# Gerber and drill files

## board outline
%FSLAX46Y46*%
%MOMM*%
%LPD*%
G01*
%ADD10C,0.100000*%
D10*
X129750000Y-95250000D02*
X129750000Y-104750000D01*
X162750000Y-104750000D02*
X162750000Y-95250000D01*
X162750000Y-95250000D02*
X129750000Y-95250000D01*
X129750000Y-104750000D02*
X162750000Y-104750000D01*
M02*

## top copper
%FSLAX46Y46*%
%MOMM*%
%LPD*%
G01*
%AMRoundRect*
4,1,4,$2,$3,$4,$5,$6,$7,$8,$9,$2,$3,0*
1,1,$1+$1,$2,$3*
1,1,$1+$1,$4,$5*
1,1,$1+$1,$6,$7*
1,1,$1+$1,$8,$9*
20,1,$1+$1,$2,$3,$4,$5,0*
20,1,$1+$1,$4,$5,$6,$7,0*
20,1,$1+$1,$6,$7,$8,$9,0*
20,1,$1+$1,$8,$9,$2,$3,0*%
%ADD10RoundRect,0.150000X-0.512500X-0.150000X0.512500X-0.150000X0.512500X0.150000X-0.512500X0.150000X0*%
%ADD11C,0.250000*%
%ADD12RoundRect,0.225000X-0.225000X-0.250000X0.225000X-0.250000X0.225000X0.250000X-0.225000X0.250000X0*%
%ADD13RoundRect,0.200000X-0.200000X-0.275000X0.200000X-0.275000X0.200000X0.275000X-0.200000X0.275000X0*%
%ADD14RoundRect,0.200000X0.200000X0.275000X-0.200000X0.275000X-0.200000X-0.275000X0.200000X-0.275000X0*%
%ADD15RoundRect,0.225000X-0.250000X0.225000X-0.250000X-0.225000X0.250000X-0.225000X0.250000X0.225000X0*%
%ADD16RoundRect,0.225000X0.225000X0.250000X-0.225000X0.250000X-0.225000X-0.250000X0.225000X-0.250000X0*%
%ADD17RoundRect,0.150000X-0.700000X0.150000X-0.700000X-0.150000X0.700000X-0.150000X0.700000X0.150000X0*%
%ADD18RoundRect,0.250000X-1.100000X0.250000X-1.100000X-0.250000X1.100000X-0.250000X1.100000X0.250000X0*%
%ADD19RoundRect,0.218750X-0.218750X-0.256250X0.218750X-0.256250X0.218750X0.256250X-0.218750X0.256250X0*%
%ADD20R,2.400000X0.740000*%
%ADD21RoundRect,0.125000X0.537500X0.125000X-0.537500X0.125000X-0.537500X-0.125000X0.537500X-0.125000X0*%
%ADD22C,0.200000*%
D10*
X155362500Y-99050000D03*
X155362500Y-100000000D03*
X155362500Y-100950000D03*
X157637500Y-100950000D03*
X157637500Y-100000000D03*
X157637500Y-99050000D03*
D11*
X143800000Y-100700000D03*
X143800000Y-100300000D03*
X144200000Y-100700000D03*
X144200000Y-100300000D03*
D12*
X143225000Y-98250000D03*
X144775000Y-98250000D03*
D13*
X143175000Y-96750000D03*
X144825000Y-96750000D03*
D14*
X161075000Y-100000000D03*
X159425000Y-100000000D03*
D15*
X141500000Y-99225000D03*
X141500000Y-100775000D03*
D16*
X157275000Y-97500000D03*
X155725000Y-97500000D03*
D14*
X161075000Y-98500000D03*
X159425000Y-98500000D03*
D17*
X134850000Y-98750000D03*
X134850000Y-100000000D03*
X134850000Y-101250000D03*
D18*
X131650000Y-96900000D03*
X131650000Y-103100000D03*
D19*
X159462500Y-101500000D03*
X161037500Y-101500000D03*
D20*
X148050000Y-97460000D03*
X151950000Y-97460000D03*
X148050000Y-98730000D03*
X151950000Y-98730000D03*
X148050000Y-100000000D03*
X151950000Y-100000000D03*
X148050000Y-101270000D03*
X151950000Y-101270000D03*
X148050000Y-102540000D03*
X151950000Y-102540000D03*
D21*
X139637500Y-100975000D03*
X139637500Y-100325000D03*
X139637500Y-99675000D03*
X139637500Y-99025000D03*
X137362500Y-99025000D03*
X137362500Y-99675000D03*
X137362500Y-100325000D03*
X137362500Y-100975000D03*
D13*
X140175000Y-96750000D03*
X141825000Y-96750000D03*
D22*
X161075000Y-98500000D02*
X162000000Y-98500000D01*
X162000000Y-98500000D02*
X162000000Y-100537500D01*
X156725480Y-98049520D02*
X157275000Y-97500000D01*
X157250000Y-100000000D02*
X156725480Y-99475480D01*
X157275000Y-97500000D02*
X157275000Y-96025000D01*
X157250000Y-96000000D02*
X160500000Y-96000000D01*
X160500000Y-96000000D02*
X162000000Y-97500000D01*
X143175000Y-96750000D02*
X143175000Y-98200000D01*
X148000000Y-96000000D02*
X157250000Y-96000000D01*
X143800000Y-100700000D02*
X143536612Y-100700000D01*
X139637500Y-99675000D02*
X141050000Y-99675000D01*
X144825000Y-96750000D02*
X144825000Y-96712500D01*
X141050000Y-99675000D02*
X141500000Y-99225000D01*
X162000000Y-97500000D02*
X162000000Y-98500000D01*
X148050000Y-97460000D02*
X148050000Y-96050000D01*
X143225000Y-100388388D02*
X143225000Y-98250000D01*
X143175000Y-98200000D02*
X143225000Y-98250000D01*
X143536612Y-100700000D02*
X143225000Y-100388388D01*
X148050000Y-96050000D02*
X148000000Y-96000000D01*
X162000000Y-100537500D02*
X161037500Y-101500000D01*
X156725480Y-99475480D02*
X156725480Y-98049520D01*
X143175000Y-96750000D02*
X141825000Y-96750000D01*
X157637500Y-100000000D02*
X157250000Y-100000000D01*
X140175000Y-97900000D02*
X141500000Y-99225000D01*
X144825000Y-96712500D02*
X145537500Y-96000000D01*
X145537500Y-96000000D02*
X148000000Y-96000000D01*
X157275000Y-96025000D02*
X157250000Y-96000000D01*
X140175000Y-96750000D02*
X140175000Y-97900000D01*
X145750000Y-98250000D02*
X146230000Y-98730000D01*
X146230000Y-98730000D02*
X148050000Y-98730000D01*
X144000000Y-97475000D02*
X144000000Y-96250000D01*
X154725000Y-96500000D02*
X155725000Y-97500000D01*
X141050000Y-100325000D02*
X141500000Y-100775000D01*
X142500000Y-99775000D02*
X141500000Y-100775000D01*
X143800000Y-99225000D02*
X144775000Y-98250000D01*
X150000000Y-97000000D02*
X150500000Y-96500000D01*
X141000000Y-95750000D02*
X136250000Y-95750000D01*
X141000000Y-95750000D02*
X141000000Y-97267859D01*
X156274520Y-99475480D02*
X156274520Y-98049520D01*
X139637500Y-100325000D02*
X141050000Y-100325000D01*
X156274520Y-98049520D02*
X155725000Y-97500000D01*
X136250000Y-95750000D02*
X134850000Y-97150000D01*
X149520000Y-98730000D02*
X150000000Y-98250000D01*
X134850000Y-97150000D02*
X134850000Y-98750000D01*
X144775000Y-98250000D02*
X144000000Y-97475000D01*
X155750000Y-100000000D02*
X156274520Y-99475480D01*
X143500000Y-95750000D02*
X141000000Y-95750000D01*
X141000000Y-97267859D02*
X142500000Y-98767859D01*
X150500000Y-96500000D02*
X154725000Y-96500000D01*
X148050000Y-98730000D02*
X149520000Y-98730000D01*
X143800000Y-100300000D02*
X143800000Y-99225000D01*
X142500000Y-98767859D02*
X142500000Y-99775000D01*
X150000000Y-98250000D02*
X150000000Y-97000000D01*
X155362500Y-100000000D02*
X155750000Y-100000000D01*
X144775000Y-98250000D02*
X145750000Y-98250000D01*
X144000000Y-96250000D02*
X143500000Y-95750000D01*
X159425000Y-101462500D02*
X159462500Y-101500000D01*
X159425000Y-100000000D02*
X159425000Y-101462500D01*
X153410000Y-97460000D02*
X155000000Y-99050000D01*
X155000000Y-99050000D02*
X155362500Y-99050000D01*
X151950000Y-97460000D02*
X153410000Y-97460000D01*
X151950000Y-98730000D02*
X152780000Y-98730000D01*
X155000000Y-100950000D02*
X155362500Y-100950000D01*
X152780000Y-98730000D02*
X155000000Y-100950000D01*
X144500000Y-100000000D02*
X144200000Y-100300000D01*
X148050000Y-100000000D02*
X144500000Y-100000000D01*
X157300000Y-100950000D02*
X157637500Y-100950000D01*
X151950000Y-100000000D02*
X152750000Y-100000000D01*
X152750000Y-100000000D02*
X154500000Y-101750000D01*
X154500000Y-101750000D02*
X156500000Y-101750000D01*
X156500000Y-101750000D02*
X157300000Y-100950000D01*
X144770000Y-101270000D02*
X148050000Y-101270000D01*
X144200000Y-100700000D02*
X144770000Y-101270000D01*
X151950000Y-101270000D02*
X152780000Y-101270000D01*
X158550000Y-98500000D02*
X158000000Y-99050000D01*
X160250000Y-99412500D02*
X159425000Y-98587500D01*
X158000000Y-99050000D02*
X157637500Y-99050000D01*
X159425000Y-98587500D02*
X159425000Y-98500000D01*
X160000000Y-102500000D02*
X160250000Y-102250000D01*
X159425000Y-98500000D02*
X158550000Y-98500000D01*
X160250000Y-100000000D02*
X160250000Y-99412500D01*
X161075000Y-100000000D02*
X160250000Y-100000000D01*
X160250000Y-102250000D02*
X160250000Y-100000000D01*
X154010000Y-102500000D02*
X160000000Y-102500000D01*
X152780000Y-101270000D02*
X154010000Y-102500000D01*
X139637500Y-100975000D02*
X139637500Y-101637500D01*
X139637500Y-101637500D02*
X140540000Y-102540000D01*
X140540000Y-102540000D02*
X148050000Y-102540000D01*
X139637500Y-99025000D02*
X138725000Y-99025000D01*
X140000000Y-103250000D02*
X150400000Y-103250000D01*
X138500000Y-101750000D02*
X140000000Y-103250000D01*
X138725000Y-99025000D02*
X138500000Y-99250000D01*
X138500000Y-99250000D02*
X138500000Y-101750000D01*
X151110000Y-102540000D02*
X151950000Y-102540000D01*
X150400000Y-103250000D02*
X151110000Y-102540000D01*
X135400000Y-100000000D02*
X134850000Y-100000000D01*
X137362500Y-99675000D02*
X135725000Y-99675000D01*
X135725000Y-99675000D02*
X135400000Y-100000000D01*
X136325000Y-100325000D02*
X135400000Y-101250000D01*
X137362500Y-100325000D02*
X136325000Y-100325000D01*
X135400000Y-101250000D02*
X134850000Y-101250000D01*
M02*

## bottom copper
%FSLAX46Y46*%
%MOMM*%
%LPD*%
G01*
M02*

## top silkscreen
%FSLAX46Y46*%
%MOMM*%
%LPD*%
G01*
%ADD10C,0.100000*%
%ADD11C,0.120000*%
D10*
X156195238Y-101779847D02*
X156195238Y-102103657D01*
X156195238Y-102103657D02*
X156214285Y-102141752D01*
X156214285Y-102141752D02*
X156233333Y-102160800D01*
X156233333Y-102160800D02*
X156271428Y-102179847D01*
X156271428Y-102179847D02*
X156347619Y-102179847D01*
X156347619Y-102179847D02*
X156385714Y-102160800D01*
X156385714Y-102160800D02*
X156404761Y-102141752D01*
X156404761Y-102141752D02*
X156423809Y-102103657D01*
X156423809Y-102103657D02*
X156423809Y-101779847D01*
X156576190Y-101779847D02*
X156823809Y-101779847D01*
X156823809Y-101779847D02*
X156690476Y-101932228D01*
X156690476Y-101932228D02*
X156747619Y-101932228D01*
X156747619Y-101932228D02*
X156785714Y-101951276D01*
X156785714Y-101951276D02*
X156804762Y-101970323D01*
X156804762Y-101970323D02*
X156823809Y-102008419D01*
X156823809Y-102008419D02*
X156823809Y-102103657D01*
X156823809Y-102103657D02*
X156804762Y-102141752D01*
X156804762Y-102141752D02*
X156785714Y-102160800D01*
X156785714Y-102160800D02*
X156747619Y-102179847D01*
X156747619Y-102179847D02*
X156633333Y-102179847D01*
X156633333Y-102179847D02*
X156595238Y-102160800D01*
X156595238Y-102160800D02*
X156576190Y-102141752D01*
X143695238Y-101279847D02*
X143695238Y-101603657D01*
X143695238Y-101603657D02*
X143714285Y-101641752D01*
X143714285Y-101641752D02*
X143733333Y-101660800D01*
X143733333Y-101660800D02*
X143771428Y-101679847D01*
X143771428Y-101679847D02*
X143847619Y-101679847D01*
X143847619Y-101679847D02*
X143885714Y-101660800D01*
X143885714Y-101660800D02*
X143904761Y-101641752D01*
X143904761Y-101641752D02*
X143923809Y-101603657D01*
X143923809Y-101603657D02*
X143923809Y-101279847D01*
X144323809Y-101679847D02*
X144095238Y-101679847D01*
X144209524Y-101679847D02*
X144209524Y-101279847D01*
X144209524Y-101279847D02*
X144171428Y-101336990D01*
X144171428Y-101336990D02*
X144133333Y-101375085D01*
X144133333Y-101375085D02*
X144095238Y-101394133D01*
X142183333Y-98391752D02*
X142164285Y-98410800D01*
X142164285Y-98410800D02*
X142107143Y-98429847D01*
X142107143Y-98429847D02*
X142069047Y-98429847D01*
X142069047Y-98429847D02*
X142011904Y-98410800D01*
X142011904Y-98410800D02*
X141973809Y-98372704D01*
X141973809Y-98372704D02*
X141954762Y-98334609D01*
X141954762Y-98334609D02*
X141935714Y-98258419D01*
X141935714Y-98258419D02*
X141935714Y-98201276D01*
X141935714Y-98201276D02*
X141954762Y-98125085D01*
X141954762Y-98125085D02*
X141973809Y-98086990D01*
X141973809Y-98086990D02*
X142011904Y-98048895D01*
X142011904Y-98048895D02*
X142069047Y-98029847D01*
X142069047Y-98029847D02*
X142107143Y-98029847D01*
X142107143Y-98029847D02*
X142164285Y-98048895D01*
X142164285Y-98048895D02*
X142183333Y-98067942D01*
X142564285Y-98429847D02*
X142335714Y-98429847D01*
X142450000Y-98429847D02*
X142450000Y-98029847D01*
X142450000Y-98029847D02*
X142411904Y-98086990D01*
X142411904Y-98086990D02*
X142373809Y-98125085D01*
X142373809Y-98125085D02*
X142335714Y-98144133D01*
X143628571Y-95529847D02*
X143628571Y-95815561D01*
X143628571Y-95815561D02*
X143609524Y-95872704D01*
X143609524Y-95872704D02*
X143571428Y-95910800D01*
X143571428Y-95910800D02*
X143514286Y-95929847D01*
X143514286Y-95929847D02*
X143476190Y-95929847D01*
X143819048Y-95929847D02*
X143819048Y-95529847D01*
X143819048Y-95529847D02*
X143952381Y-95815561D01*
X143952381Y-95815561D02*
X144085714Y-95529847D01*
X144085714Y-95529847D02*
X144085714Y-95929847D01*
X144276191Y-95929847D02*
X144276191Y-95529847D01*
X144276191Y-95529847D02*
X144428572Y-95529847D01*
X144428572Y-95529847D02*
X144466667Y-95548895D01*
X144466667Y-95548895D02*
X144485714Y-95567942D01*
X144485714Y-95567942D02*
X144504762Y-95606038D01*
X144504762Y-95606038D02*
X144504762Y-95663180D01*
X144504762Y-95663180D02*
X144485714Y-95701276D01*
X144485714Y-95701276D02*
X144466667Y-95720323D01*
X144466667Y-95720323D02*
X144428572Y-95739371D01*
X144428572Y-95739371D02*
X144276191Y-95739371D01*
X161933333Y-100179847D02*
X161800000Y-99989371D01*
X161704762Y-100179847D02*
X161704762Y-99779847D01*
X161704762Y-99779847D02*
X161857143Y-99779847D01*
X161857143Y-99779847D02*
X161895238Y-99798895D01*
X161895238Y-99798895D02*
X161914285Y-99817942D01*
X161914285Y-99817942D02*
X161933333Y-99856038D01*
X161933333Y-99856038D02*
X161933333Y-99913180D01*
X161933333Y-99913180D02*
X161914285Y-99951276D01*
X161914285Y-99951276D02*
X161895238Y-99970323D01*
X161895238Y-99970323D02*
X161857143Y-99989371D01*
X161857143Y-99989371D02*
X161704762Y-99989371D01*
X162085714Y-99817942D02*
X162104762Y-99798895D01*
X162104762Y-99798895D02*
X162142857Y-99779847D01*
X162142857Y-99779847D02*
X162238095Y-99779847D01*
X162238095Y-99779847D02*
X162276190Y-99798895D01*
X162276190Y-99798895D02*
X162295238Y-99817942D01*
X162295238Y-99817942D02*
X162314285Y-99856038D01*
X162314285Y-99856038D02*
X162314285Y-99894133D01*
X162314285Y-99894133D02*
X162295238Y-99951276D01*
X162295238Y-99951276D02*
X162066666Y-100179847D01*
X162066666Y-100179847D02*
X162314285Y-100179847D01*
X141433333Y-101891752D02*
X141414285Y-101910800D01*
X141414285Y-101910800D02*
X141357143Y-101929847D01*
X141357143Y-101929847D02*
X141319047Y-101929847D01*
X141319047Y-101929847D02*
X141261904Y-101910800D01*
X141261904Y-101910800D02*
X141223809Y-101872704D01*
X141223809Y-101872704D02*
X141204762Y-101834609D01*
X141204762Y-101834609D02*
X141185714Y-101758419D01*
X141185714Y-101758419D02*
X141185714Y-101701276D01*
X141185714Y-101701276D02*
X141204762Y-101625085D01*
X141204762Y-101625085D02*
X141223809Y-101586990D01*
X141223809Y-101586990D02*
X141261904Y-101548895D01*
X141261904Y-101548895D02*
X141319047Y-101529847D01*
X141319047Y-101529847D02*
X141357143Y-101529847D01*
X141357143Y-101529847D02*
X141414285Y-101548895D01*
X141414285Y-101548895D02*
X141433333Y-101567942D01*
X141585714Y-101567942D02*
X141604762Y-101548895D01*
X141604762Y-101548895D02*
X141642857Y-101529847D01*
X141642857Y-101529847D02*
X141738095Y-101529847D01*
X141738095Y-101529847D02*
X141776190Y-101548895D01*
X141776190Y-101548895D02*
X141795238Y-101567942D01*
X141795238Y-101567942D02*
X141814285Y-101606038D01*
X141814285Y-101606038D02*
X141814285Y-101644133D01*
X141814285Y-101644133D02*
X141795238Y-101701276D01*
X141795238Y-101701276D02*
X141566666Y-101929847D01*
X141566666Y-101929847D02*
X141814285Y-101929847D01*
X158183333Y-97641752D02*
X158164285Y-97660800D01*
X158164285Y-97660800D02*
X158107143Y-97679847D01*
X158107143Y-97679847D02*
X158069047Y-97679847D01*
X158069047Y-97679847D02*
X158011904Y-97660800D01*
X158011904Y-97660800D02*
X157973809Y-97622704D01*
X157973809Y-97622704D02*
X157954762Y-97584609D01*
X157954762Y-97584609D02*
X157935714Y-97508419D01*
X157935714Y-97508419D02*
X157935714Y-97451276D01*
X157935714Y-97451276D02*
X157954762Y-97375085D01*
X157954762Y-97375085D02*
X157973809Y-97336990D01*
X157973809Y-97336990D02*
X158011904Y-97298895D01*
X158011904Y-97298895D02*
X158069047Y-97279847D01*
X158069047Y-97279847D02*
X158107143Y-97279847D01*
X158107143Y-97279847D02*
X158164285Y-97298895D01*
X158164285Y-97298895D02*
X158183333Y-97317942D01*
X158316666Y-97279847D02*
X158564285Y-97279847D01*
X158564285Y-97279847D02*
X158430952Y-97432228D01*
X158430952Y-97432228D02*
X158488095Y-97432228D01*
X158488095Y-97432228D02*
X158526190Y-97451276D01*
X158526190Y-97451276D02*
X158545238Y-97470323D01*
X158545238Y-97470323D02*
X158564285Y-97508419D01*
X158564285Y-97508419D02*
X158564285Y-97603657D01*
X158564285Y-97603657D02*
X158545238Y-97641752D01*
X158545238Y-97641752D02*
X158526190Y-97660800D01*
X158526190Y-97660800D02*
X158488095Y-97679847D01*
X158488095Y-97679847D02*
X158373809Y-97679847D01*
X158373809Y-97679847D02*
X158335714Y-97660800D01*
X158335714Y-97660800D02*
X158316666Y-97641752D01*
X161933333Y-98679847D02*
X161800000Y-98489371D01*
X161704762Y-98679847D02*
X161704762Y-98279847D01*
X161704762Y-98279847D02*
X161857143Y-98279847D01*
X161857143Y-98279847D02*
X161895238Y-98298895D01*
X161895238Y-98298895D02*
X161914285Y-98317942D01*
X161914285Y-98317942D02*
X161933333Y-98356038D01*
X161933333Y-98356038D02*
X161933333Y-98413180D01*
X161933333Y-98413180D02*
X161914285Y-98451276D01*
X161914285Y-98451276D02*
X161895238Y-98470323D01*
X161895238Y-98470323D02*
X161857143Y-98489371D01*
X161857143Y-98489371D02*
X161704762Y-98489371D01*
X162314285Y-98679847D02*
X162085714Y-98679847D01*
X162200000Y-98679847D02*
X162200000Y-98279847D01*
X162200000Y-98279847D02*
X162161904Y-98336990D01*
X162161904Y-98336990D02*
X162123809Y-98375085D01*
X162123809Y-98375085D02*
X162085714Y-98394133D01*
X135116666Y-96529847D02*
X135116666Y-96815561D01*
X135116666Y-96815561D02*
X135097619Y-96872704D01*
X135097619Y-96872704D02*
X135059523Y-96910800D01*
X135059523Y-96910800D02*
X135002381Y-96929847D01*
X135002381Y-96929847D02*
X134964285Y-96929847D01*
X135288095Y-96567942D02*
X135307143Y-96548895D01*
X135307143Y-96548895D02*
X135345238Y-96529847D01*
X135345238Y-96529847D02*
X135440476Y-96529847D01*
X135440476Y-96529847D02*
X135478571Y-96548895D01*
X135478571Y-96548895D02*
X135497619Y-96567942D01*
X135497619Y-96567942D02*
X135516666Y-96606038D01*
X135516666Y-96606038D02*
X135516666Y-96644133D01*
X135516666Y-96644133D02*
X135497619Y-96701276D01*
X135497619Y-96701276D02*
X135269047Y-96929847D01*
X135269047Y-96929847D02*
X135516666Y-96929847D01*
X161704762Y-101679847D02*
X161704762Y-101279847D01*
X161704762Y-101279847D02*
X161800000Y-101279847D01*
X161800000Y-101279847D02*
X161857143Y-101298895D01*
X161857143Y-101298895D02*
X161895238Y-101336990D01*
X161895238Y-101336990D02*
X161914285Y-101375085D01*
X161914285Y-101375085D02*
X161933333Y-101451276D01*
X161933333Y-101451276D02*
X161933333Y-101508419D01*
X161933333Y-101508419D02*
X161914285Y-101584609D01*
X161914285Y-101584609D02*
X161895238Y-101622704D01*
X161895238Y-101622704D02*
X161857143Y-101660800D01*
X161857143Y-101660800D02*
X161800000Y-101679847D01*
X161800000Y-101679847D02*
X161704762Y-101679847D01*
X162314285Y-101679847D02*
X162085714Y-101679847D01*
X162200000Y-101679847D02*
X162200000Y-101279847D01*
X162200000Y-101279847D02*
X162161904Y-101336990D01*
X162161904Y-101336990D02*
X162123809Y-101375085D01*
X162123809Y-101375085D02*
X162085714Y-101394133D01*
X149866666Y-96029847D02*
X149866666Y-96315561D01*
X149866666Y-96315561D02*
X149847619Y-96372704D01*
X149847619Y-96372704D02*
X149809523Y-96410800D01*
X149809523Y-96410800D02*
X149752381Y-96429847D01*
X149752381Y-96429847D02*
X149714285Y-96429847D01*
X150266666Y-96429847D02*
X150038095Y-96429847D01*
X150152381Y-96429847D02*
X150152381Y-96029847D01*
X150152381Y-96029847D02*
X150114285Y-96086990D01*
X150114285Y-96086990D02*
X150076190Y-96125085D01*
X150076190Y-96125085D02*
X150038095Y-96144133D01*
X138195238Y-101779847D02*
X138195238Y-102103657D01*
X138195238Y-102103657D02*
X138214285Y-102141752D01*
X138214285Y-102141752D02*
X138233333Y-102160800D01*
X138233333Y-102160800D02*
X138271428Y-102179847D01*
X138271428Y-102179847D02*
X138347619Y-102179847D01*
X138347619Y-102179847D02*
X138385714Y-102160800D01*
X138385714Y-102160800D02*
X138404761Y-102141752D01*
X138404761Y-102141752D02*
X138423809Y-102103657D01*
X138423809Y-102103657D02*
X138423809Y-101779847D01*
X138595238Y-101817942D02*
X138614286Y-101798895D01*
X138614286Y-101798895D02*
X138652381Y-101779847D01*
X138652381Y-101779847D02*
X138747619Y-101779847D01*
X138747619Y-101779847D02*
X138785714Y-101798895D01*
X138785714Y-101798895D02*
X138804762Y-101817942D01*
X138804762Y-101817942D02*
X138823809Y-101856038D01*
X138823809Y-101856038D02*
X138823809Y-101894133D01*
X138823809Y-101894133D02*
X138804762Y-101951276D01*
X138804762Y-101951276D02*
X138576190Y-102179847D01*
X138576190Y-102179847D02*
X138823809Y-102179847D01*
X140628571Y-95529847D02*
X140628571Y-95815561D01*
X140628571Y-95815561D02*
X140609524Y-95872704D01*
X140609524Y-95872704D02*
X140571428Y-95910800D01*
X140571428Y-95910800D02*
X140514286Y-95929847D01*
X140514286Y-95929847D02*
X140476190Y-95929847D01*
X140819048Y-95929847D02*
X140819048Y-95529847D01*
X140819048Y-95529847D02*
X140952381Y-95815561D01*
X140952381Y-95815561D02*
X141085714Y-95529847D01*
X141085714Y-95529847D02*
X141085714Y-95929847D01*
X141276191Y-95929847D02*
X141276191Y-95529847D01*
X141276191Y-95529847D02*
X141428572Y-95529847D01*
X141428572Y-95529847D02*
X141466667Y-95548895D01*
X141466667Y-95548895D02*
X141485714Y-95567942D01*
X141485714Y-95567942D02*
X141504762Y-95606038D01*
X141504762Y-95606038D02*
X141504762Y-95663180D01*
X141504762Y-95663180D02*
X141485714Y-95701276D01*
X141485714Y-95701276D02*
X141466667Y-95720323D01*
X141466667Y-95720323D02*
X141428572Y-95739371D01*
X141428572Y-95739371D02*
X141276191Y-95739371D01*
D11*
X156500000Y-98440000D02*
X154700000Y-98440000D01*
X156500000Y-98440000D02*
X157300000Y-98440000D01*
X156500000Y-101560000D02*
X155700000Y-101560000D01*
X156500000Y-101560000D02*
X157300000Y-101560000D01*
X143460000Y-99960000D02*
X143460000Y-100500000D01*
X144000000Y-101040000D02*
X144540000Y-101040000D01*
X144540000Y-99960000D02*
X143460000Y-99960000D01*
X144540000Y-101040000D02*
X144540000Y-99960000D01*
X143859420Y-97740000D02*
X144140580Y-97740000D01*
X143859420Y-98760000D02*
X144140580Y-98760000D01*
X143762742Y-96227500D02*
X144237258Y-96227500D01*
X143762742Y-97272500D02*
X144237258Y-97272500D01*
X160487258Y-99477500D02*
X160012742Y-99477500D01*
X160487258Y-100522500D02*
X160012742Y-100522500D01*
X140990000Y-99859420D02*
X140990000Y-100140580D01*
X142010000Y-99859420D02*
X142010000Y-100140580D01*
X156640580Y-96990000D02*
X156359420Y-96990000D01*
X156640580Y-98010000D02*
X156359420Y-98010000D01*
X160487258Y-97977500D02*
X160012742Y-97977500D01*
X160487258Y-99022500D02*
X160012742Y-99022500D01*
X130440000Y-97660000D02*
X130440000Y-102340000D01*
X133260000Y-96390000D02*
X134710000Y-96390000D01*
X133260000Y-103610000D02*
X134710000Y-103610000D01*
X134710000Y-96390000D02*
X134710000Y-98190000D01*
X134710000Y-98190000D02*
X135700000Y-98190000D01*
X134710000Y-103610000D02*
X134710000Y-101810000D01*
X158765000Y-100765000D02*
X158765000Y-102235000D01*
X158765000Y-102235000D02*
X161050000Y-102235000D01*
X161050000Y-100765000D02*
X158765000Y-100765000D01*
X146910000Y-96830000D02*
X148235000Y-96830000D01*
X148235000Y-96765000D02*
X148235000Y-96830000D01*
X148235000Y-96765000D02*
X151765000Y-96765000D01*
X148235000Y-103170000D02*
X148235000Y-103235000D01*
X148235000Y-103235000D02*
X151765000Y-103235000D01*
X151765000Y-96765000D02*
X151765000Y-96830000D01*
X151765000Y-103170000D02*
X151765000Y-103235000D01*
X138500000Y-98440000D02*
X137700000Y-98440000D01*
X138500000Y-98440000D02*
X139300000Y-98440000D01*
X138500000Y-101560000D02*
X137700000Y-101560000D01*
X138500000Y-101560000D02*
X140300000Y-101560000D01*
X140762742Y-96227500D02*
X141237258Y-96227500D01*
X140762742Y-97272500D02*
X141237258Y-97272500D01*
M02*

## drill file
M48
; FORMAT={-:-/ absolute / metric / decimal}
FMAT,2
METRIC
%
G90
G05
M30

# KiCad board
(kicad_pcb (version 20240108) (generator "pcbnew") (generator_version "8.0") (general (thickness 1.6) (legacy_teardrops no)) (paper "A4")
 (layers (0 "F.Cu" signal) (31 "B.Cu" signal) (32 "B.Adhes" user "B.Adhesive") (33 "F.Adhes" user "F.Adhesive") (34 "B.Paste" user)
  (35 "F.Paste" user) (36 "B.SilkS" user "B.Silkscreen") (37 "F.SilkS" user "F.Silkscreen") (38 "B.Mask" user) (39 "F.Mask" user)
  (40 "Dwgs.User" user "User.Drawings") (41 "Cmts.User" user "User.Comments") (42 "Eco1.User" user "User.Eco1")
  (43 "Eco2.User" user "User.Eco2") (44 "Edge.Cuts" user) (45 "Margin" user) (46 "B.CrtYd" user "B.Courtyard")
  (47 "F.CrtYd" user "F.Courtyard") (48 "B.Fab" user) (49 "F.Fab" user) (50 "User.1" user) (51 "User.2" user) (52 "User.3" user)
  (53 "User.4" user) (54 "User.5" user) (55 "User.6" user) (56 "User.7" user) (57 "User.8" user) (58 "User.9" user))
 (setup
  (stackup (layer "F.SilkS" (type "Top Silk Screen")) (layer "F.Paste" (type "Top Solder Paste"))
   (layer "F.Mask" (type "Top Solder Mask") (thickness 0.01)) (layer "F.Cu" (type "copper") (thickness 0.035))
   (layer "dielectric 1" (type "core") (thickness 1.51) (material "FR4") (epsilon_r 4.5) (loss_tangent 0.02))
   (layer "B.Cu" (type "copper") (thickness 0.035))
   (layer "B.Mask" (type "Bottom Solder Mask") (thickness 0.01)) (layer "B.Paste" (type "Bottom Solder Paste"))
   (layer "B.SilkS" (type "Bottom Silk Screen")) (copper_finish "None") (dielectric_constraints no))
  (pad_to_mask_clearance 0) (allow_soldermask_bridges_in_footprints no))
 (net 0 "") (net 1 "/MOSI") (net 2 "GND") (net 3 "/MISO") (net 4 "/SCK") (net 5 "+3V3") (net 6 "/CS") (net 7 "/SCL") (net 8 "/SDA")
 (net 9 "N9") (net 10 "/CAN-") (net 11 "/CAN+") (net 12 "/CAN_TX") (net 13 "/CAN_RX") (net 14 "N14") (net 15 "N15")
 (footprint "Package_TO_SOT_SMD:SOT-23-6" (layer "F.Cu") (at 156.5 100)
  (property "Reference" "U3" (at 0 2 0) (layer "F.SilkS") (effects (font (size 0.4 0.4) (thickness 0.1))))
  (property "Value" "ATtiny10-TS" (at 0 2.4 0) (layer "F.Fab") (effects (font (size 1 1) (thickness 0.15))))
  (fp_line (start 0 -1.56) (end -1.8 -1.56) (stroke (width 0.12) (type solid)) (layer "F.SilkS"))
  (fp_line (start 0 -1.56) (end 0.8 -1.56) (stroke (width 0.12) (type solid)) (layer "F.SilkS"))
  (fp_line (start 0 1.56) (end -0.8 1.56) (stroke (width 0.12) (type solid)) (layer "F.SilkS"))
  (fp_line (start 0 1.56) (end 0.8 1.56) (stroke (width 0.12) (type solid)) (layer "F.SilkS"))
  (pad "1" smd roundrect (at -1.1375 -0.95) (size 1.325 0.6) (layers "F.Cu" "F.Paste" "F.Mask") (roundrect_rratio 0.25) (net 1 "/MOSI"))
  (pad "2" smd roundrect (at -1.1375 0) (size 1.325 0.6) (layers "F.Cu" "F.Paste" "F.Mask") (roundrect_rratio 0.25) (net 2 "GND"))
  (pad "3" smd roundrect (at -1.1375 0.95) (size 1.325 0.6) (layers "F.Cu" "F.Paste" "F.Mask") (roundrect_rratio 0.25) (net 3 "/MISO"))
  (pad "4" smd roundrect (at 1.1375 0.95) (size 1.325 0.6) (layers "F.Cu" "F.Paste" "F.Mask") (roundrect_rratio 0.25) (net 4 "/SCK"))
  (pad "5" smd roundrect (at 1.1375 0) (size 1.325 0.6) (layers "F.Cu" "F.Paste" "F.Mask") (roundrect_rratio 0.25) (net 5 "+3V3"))
  (pad "6" smd roundrect (at 1.1375 -0.95) (size 1.325 0.6) (layers "F.Cu" "F.Paste" "F.Mask") (roundrect_rratio 0.25) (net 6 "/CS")))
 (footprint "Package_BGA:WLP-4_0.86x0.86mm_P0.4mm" (layer "F.Cu") (at 144 100.5 90)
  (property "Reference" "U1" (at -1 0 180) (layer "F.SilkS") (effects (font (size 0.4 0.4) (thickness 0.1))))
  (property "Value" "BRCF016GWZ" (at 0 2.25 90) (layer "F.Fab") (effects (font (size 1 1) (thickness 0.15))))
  (fp_line (start 0.54 -0.54) (end 0 -0.54) (stroke (width 0.12) (type solid)) (layer "F.SilkS"))
  (fp_line (start -0.54 0) (end -0.54 0.54) (stroke (width 0.12) (type solid)) (layer "F.SilkS"))
  (fp_line (start 0.54 0.54) (end 0.54 -0.54) (stroke (width 0.12) (type solid)) (layer "F.SilkS"))
  (fp_line (start -0.54 0.54) (end 0.54 0.54) (stroke (width 0.12) (type solid)) (layer "F.SilkS"))
  (pad "A1" smd circle (at -0.2 -0.2 90) (size 0.25 0.25) (layers "F.Cu" "F.Paste" "F.Mask") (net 5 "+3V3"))
  (pad "A2" smd circle (at 0.2 -0.2 90) (size 0.25 0.25) (layers "F.Cu" "F.Paste" "F.Mask") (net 2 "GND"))
  (pad "B1" smd circle (at -0.2 0.2 90) (size 0.25 0.25) (layers "F.Cu" "F.Paste" "F.Mask") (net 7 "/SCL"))
  (pad "B2" smd circle (at 0.2 0.2 90) (size 0.25 0.25) (layers "F.Cu" "F.Paste" "F.Mask") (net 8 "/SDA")))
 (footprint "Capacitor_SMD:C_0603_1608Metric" (layer "F.Cu") (at 144 98.25)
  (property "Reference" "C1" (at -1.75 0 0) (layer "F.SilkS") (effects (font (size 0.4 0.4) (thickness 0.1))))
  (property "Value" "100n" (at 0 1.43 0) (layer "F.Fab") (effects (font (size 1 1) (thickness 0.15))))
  (fp_line (start -0.14058 -0.51) (end 0.14058 -0.51) (stroke (width 0.12) (type solid)) (layer "F.SilkS"))
  (fp_line (start -0.14058 0.51) (end 0.14058 0.51) (stroke (width 0.12) (type solid)) (layer "F.SilkS"))
  (pad "1" smd roundrect (at -0.775 0) (size 0.9 0.95) (layers "F.Cu" "F.Paste" "F.Mask") (roundrect_rratio 0.25) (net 5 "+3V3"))
  (pad "2" smd roundrect (at 0.775 0) (size 0.9 0.95) (layers "F.Cu" "F.Paste" "F.Mask") (roundrect_rratio 0.25) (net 2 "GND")))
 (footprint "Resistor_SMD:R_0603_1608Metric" (layer "F.Cu") (at 144 96.75)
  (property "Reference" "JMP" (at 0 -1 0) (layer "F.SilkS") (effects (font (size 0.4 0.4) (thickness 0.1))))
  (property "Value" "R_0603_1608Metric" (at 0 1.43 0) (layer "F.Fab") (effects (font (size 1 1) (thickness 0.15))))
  (fp_line (start -0.237258 -0.5225) (end 0.237258 -0.5225) (stroke (width 0.12) (type solid)) (layer "F.SilkS"))
  (fp_line (start -0.237258 0.5225) (end 0.237258 0.5225) (stroke (width 0.12) (type solid)) (layer "F.SilkS"))
  (pad "1" smd roundrect (at -0.825 0) (size 0.8 0.95) (layers "F.Cu" "F.Paste" "F.Mask") (roundrect_rratio 0.25) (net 5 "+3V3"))
  (pad "2" smd roundrect (at 0.825 0) (size 0.8 0.95) (layers "F.Cu" "F.Paste" "F.Mask") (roundrect_rratio 0.25) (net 5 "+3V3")))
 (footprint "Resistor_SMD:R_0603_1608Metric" (layer "F.Cu") (at 160.25 100 180)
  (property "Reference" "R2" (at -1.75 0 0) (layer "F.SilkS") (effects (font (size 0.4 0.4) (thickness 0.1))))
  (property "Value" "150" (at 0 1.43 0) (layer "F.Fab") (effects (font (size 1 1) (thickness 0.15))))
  (fp_line (start -0.237258 0.5225) (end 0.237258 0.5225) (stroke (width 0.12) (type solid)) (layer "F.SilkS"))
  (fp_line (start -0.237258 -0.5225) (end 0.237258 -0.5225) (stroke (width 0.12) (type solid)) (layer "F.SilkS"))
  (pad "1" smd roundrect (at -0.825 0 180) (size 0.8 0.95) (layers "F.Cu" "F.Paste" "F.Mask") (roundrect_rratio 0.25) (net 6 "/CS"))
  (pad "2" smd roundrect (at 0.825 0 180) (size 0.8 0.95) (layers "F.Cu" "F.Paste" "F.Mask") (roundrect_rratio 0.25) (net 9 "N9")))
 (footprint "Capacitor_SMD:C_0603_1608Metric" (layer "F.Cu") (at 141.5 100 -90)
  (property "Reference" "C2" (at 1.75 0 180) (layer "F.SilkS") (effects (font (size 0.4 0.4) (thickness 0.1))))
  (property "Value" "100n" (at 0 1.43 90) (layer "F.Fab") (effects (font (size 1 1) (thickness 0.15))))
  (fp_line (start -0.14058 0.51) (end 0.14058 0.51) (stroke (width 0.12) (type solid)) (layer "F.SilkS"))
  (fp_line (start -0.14058 -0.51) (end 0.14058 -0.51) (stroke (width 0.12) (type solid)) (layer "F.SilkS"))
  (pad "1" smd roundrect (at -0.775 0 270) (size 0.9 0.95) (layers "F.Cu" "F.Paste" "F.Mask") (roundrect_rratio 0.25) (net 5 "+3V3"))
  (pad "2" smd roundrect (at 0.775 0 270) (size 0.9 0.95) (layers "F.Cu" "F.Paste" "F.Mask") (roundrect_rratio 0.25) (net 2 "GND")))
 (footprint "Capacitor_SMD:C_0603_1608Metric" (layer "F.Cu") (at 156.5 97.5 180)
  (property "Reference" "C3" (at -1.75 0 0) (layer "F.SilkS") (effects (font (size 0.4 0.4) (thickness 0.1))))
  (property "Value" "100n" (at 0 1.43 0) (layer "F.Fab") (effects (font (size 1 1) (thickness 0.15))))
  (fp_line (start -0.14058 0.51) (end 0.14058 0.51) (stroke (width 0.12) (type solid)) (layer "F.SilkS"))
  (fp_line (start -0.14058 -0.51) (end 0.14058 -0.51) (stroke (width 0.12) (type solid)) (layer "F.SilkS"))
  (pad "1" smd roundrect (at -0.775 0 180) (size 0.9 0.95) (layers "F.Cu" "F.Paste" "F.Mask") (roundrect_rratio 0.25) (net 5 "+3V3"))
  (pad "2" smd roundrect (at 0.775 0 180) (size 0.9 0.95) (layers "F.Cu" "F.Paste" "F.Mask") (roundrect_rratio 0.25) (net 2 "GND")))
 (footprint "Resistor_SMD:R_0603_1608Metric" (layer "F.Cu") (at 160.25 98.5 180)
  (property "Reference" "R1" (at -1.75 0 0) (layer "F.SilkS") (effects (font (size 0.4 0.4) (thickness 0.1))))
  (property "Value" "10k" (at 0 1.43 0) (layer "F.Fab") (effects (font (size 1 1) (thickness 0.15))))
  (fp_line (start -0.237258 0.5225) (end 0.237258 0.5225) (stroke (width 0.12) (type solid)) (layer "F.SilkS"))
  (fp_line (start -0.237258 -0.5225) (end 0.237258 -0.5225) (stroke (width 0.12) (type solid)) (layer "F.SilkS"))
  (pad "1" smd roundrect (at -0.825 0 180) (size 0.8 0.95) (layers "F.Cu" "F.Paste" "F.Mask") (roundrect_rratio 0.25) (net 5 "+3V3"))
  (pad "2" smd roundrect (at 0.825 0 180) (size 0.8 0.95) (layers "F.Cu" "F.Paste" "F.Mask") (roundrect_rratio 0.25) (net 6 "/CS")))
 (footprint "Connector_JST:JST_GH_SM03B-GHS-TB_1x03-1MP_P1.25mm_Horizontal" (layer "F.Cu") (at 133 100 -90)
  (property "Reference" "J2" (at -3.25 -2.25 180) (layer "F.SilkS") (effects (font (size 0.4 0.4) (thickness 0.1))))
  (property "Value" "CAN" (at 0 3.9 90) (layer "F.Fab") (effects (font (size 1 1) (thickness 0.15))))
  (fp_line (start -2.34 2.56) (end 2.34 2.56) (stroke (width 0.12) (type solid)) (layer "F.SilkS"))
  (fp_line (start -3.61 -0.26) (end -3.61 -1.71) (stroke (width 0.12) (type solid)) (layer "F.SilkS"))
  (fp_line (start 3.61 -0.26) (end 3.61 -1.71) (stroke (width 0.12) (type solid)) (layer "F.SilkS"))
  (fp_line (start -3.61 -1.71) (end -1.81 -1.71) (stroke (width 0.12) (type solid)) (layer "F.SilkS"))
  (fp_line (start -1.81 -1.71) (end -1.81 -2.7) (stroke (width 0.12) (type solid)) (layer "F.SilkS"))
  (fp_line (start 3.61 -1.71) (end 1.81 -1.71) (stroke (width 0.12) (type solid)) (layer "F.SilkS"))
  (pad "1" smd roundrect (at -1.25 -1.85 270) (size 0.6 1.7) (layers "F.Cu" "F.Paste" "F.Mask") (roundrect_rratio 0.25) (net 2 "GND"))
  (pad "2" smd roundrect (at 0 -1.85 270) (size 0.6 1.7) (layers "F.Cu" "F.Paste" "F.Mask") (roundrect_rratio 0.25) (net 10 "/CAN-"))
  (pad "3" smd roundrect (at 1.25 -1.85 270) (size 0.6 1.7) (layers "F.Cu" "F.Paste" "F.Mask") (roundrect_rratio 0.25) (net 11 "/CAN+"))
  (pad "MP" smd roundrect (at -3.1 1.35 270) (size 1 2.7) (layers "F.Cu" "F.Paste" "F.Mask") (roundrect_rratio 0.25))
  (pad "MP" smd roundrect (at 3.1 1.35 270) (size 1 2.7) (layers "F.Cu" "F.Paste" "F.Mask") (roundrect_rratio 0.25)))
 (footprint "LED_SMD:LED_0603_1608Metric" (layer "F.Cu") (at 160.25 101.5)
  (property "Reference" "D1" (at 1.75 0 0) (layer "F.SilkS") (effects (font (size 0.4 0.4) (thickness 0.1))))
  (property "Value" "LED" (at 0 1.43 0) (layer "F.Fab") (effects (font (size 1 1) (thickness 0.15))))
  (fp_line (start -1.485 -0.735) (end -1.485 0.735) (stroke (width 0.12) (type solid)) (layer "F.SilkS"))
  (fp_line (start -1.485 0.735) (end 0.8 0.735) (stroke (width 0.12) (type solid)) (layer "F.SilkS"))
  (fp_line (start 0.8 -0.735) (end -1.485 -0.735) (stroke (width 0.12) (type solid)) (layer "F.SilkS"))
  (pad "1" smd roundrect (at -0.7875 0) (size 0.875 0.95) (layers "F.Cu" "F.Paste" "F.Mask") (roundrect_rratio 0.25) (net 9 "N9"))
  (pad "2" smd roundrect (at 0.7875 0) (size 0.875 0.95) (layers "F.Cu" "F.Paste" "F.Mask") (roundrect_rratio 0.25) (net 5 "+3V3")))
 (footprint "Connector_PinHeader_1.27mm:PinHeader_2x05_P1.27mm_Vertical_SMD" (layer "F.Cu") (at 150 100)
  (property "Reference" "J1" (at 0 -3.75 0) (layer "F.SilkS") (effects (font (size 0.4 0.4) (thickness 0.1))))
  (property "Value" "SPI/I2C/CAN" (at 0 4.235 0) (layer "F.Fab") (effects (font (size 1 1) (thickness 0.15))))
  (fp_line (start -3.09 -3.17) (end -1.765 -3.17) (stroke (width 0.12) (type solid)) (layer "F.SilkS"))
  (fp_line (start -1.765 -3.235) (end -1.765 -3.17) (stroke (width 0.12) (type solid)) (layer "F.SilkS"))
  (fp_line (start -1.765 -3.235) (end 1.765 -3.235) (stroke (width 0.12) (type solid)) (layer "F.SilkS"))
  (fp_line (start -1.765 3.17) (end -1.765 3.235) (stroke (width 0.12) (type solid)) (layer "F.SilkS"))
  (fp_line (start -1.765 3.235) (end 1.765 3.235) (stroke (width 0.12) (type solid)) (layer "F.SilkS"))
  (fp_line (start 1.765 -3.235) (end 1.765 -3.17) (stroke (width 0.12) (type solid)) (layer "F.SilkS"))
  (fp_line (start 1.765 3.17) (end 1.765 3.235) (stroke (width 0.12) (type solid)) (layer "F.SilkS"))
  (pad "1" smd rect (at -1.95 -2.54) (size 2.4 0.74) (layers "F.Cu" "F.Paste" "F.Mask") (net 5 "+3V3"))
  (pad "2" smd rect (at 1.95 -2.54) (size 2.4 0.74) (layers "F.Cu" "F.Paste" "F.Mask") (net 1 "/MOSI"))
  (pad "3" smd rect (at -1.95 -1.27) (size 2.4 0.74) (layers "F.Cu" "F.Paste" "F.Mask") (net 2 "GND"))
  (pad "4" smd rect (at 1.95 -1.27) (size 2.4 0.74) (layers "F.Cu" "F.Paste" "F.Mask") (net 3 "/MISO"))
  (pad "5" smd rect (at -1.95 0) (size 2.4 0.74) (layers "F.Cu" "F.Paste" "F.Mask") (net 8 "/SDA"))
  (pad "6" smd rect (at 1.95 0) (size 2.4 0.74) (layers "F.Cu" "F.Paste" "F.Mask") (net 4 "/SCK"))
  (pad "7" smd rect (at -1.95 1.27) (size 2.4 0.74) (layers "F.Cu" "F.Paste" "F.Mask") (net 7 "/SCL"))
  (pad "8" smd rect (at 1.95 1.27) (size 2.4 0.74) (layers "F.Cu" "F.Paste" "F.Mask") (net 6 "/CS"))
  (pad "9" smd rect (at -1.95 2.54) (size 2.4 0.74) (layers "F.Cu" "F.Paste" "F.Mask") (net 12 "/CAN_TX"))
  (pad "10" smd rect (at 1.95 2.54) (size 2.4 0.74) (layers "F.Cu" "F.Paste" "F.Mask") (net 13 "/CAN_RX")))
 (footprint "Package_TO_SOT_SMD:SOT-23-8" (layer "F.Cu") (at 138.5 100 180)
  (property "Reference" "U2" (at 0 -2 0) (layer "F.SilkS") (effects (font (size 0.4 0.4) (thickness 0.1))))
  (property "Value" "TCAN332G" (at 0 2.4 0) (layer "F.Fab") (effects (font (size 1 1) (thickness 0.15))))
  (fp_line (start 0 1.56) (end 0.8 1.56) (stroke (width 0.12) (type solid)) (layer "F.SilkS"))
  (fp_line (start 0 1.56) (end -0.8 1.56) (stroke (width 0.12) (type solid)) (layer "F.SilkS"))
  (fp_line (start 0 -1.56) (end 0.8 -1.56) (stroke (width 0.12) (type solid)) (layer "F.SilkS"))
  (fp_line (start 0 -1.56) (end -1.8 -1.56) (stroke (width 0.12) (type solid)) (layer "F.SilkS"))
  (pad "1" smd roundrect (at -1.1375 -0.975 180) (size 1.325 0.5) (layers "F.Cu" "F.Paste" "F.Mask") (roundrect_rratio 0.25)
   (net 12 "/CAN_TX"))
  (pad "2" smd roundrect (at -1.1375 -0.325 180) (size 1.325 0.5) (layers "F.Cu" "F.Paste" "F.Mask") (roundrect_rratio 0.25) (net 2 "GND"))
  (pad "3" smd roundrect (at -1.1375 0.325 180) (size 1.325 0.5) (layers "F.Cu" "F.Paste" "F.Mask") (roundrect_rratio 0.25) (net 5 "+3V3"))
  (pad "4" smd roundrect (at -1.1375 0.975 180) (size 1.325 0.5) (layers "F.Cu" "F.Paste" "F.Mask") (roundrect_rratio 0.25)
   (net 13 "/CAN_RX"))
  (pad "5" smd roundrect (at 1.1375 0.975 180) (size 1.325 0.5) (layers "F.Cu" "F.Paste" "F.Mask") (roundrect_rratio 0.25) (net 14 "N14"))
  (pad "6" smd roundrect (at 1.1375 0.325 180) (size 1.325 0.5) (layers "F.Cu" "F.Paste" "F.Mask") (roundrect_rratio 0.25) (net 10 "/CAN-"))
  (pad "7" smd roundrect (at 1.1375 -0.325 180) (size 1.325 0.5) (layers "F.Cu" "F.Paste" "F.Mask") (roundrect_rratio 0.25) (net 11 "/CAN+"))
  (pad "8" smd roundrect (at 1.1375 -0.975 180) (size 1.325 0.5) (layers "F.Cu" "F.Paste" "F.Mask") (roundrect_rratio 0.25) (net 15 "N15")))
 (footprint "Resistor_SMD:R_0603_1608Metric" (layer "F.Cu") (at 141 96.75)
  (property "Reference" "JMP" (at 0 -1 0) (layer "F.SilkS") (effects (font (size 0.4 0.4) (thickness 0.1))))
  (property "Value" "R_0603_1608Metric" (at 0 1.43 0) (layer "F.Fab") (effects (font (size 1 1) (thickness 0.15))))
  (fp_line (start -0.237258 -0.5225) (end 0.237258 -0.5225) (stroke (width 0.12) (type solid)) (layer "F.SilkS"))
  (fp_line (start -0.237258 0.5225) (end 0.237258 0.5225) (stroke (width 0.12) (type solid)) (layer "F.SilkS"))
  (pad "1" smd roundrect (at -0.825 0) (size 0.8 0.95) (layers "F.Cu" "F.Paste" "F.Mask") (roundrect_rratio 0.25) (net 5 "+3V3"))
  (pad "2" smd roundrect (at 0.825 0) (size 0.8 0.95) (layers "F.Cu" "F.Paste" "F.Mask") (roundrect_rratio 0.25) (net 5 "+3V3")))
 (gr_line (start 129.75 95.25) (end 129.75 104.75) (stroke (width 0.1) (type solid)) (layer "Edge.Cuts"))
 (gr_line (start 162.75 104.75) (end 162.75 95.25) (stroke (width 0.1) (type solid)) (layer "Edge.Cuts"))
 (gr_line (start 162.75 95.25) (end 129.75 95.25) (stroke (width 0.1) (type solid)) (layer "Edge.Cuts"))
 (gr_line (start 129.75 104.75) (end 162.75 104.75) (stroke (width 0.1) (type solid)) (layer "Edge.Cuts"))
 (segment (start 161.075 98.5) (end 162 98.5) (width 0.2) (layer "F.Cu") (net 5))
 (segment (start 162 98.5) (end 162 100.5375) (width 0.2) (layer "F.Cu") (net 5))
 (segment (start 156.72548 98.04952) (end 157.275 97.5) (width 0.2) (layer "F.Cu") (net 5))
 (segment (start 157.25 100) (end 156.72548 99.47548) (width 0.2) (layer "F.Cu") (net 5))
 (segment (start 157.275 97.5) (end 157.275 96.025) (width 0.2) (layer "F.Cu") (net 5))
 (segment (start 157.25 96) (end 160.5 96) (width 0.2) (layer "F.Cu") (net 5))
 (segment (start 160.5 96) (end 162 97.5) (width 0.2) (layer "F.Cu") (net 5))
 (segment (start 143.175 96.75) (end 143.175 98.2) (width 0.2) (layer "F.Cu") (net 5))
 (segment (start 148 96) (end 157.25 96) (width 0.2) (layer "F.Cu") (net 5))
 (segment (start 143.8 100.7) (end 143.536612 100.7) (width 0.2) (layer "F.Cu") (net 5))
 (segment (start 139.6375 99.675) (end 141.05 99.675) (width 0.2) (layer "F.Cu") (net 5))
 (segment (start 144.825 96.75) (end 144.825 96.7125) (width 0.2) (layer "F.Cu") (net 5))
 (segment (start 141.05 99.675) (end 141.5 99.225) (width 0.2) (layer "F.Cu") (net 5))
 (segment (start 162 97.5) (end 162 98.5) (width 0.2) (layer "F.Cu") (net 5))
 (segment (start 148.05 97.46) (end 148.05 96.05) (width 0.2) (layer "F.Cu") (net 5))
 (segment (start 143.225 100.388388) (end 143.225 98.25) (width 0.2) (layer "F.Cu") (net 5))
 (segment (start 143.175 98.2) (end 143.225 98.25) (width 0.2) (layer "F.Cu") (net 5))
 (segment (start 143.536612 100.7) (end 143.225 100.388388) (width 0.2) (layer "F.Cu") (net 5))
 (segment (start 148.05 96.05) (end 148 96) (width 0.2) (layer "F.Cu") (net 5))
 (segment (start 162 100.5375) (end 161.0375 101.5) (width 0.2) (layer "F.Cu") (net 5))
 (segment (start 156.72548 99.47548) (end 156.72548 98.04952) (width 0.2) (layer "F.Cu") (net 5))
 (segment (start 143.175 96.75) (end 141.825 96.75) (width 0.2) (layer "F.Cu") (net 5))
 (segment (start 157.6375 100) (end 157.25 100) (width 0.2) (layer "F.Cu") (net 5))
 (segment (start 140.175 97.9) (end 141.5 99.225) (width 0.2) (layer "F.Cu") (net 5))
 (segment (start 144.825 96.7125) (end 145.5375 96) (width 0.2) (layer "F.Cu") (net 5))
 (segment (start 145.5375 96) (end 148 96) (width 0.2) (layer "F.Cu") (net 5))
 (segment (start 157.275 96.025) (end 157.25 96) (width 0.2) (layer "F.Cu") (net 5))
 (segment (start 140.175 96.75) (end 140.175 97.9) (width 0.2) (layer "F.Cu") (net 5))
 (segment (start 145.75 98.25) (end 146.23 98.73) (width 0.2) (layer "F.Cu") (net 2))
 (segment (start 146.23 98.73) (end 148.05 98.73) (width 0.2) (layer "F.Cu") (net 2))
 (segment (start 144 97.475) (end 144 96.25) (width 0.2) (layer "F.Cu") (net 2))
 (segment (start 154.725 96.5) (end 155.725 97.5) (width 0.2) (layer "F.Cu") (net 2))
 (segment (start 141.05 100.325) (end 141.5 100.775) (width 0.2) (layer "F.Cu") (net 2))
 (segment (start 142.5 99.775) (end 141.5 100.775) (width 0.2) (layer "F.Cu") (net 2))
 (segment (start 143.8 99.225) (end 144.775 98.25) (width 0.2) (layer "F.Cu") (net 2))
 (segment (start 150 97) (end 150.5 96.5) (width 0.2) (layer "F.Cu") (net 2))
 (segment (start 141 95.75) (end 136.25 95.75) (width 0.2) (layer "F.Cu") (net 2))
 (segment (start 141 95.75) (end 141 97.267859) (width 0.2) (layer "F.Cu") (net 2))
 (segment (start 156.27452 99.47548) (end 156.27452 98.04952) (width 0.2) (layer "F.Cu") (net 2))
 (segment (start 139.6375 100.325) (end 141.05 100.325) (width 0.2) (layer "F.Cu") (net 2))
 (segment (start 156.27452 98.04952) (end 155.725 97.5) (width 0.2) (layer "F.Cu") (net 2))
 (segment (start 136.25 95.75) (end 134.85 97.15) (width 0.2) (layer "F.Cu") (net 2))
 (segment (start 149.52 98.73) (end 150 98.25) (width 0.2) (layer "F.Cu") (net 2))
 (segment (start 134.85 97.15) (end 134.85 98.75) (width 0.2) (layer "F.Cu") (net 2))
 (segment (start 144.775 98.25) (end 144 97.475) (width 0.2) (layer "F.Cu") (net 2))
 (segment (start 155.75 100) (end 156.27452 99.47548) (width 0.2) (layer "F.Cu") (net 2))
 (segment (start 143.5 95.75) (end 141 95.75) (width 0.2) (layer "F.Cu") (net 2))
 (segment (start 141 97.267859) (end 142.5 98.767859) (width 0.2) (layer "F.Cu") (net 2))
 (segment (start 150.5 96.5) (end 154.725 96.5) (width 0.2) (layer "F.Cu") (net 2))
 (segment (start 148.05 98.73) (end 149.52 98.73) (width 0.2) (layer "F.Cu") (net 2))
 (segment (start 143.8 100.3) (end 143.8 99.225) (width 0.2) (layer "F.Cu") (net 2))
 (segment (start 142.5 98.767859) (end 142.5 99.775) (width 0.2) (layer "F.Cu") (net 2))
 (segment (start 150 98.25) (end 150 97) (width 0.2) (layer "F.Cu") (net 2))
 (segment (start 155.3625 100) (end 155.75 100) (width 0.2) (layer "F.Cu") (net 2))
 (segment (start 144.775 98.25) (end 145.75 98.25) (width 0.2) (layer "F.Cu") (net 2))
 (segment (start 144 96.25) (end 143.5 95.75) (width 0.2) (layer "F.Cu") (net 2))
 (segment (start 159.425 101.4625) (end 159.4625 101.5) (width 0.2) (layer "F.Cu") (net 9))
 (segment (start 159.425 100) (end 159.425 101.4625) (width 0.2) (layer "F.Cu") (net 9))
 (segment (start 153.41 97.46) (end 155 99.05) (width 0.2) (layer "F.Cu") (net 1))
 (segment (start 155 99.05) (end 155.3625 99.05) (width 0.2) (layer "F.Cu") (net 1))
 (segment (start 151.95 97.46) (end 153.41 97.46) (width 0.2) (layer "F.Cu") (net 1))
 (segment (start 151.95 98.73) (end 152.78 98.73) (width 0.2) (layer "F.Cu") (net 3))
 (segment (start 155 100.95) (end 155.3625 100.95) (width 0.2) (layer "F.Cu") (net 3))
 (segment (start 152.78 98.73) (end 155 100.95) (width 0.2) (layer "F.Cu") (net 3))
 (segment (start 144.5 100) (end 144.2 100.3) (width 0.2) (layer "F.Cu") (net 8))
 (segment (start 148.05 100) (end 144.5 100) (width 0.2) (layer "F.Cu") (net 8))
 (segment (start 157.3 100.95) (end 157.6375 100.95) (width 0.2) (layer "F.Cu") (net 4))
 (segment (start 151.95 100) (end 152.75 100) (width 0.2) (layer "F.Cu") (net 4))
 (segment (start 152.75 100) (end 154.5 101.75) (width 0.2) (layer "F.Cu") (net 4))
 (segment (start 154.5 101.75) (end 156.5 101.75) (width 0.2) (layer "F.Cu") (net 4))
 (segment (start 156.5 101.75) (end 157.3 100.95) (width 0.2) (layer "F.Cu") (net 4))
 (segment (start 144.77 101.27) (end 148.05 101.27) (width 0.2) (layer "F.Cu") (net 7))
 (segment (start 144.2 100.7) (end 144.77 101.27) (width 0.2) (layer "F.Cu") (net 7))
 (segment (start 151.95 101.27) (end 152.78 101.27) (width 0.2) (layer "F.Cu") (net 6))
 (segment (start 158.55 98.5) (end 158 99.05) (width 0.2) (layer "F.Cu") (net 6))
 (segment (start 160.25 99.4125) (end 159.425 98.5875) (width 0.2) (layer "F.Cu") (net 6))
 (segment (start 158 99.05) (end 157.6375 99.05) (width 0.2) (layer "F.Cu") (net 6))
 (segment (start 159.425 98.5875) (end 159.425 98.5) (width 0.2) (layer "F.Cu") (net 6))
 (segment (start 160 102.5) (end 160.25 102.25) (width 0.2) (layer "F.Cu") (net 6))
 (segment (start 159.425 98.5) (end 158.55 98.5) (width 0.2) (layer "F.Cu") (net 6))
 (segment (start 160.25 100) (end 160.25 99.4125) (width 0.2) (layer "F.Cu") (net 6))
 (segment (start 161.075 100) (end 160.25 100) (width 0.2) (layer "F.Cu") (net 6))
 (segment (start 160.25 102.25) (end 160.25 100) (width 0.2) (layer "F.Cu") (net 6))
 (segment (start 154.01 102.5) (end 160 102.5) (width 0.2) (layer "F.Cu") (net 6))
 (segment (start 152.78 101.27) (end 154.01 102.5) (width 0.2) (layer "F.Cu") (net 6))
 (segment (start 139.6375 100.975) (end 139.6375 101.6375) (width 0.2) (layer "F.Cu") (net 12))
 (segment (start 139.6375 101.6375) (end 140.54 102.54) (width 0.2) (layer "F.Cu") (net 12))
 (segment (start 140.54 102.54) (end 148.05 102.54) (width 0.2) (layer "F.Cu") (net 12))
 (segment (start 139.6375 99.025) (end 138.725 99.025) (width 0.2) (layer "F.Cu") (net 13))
 (segment (start 140 103.25) (end 150.4 103.25) (width 0.2) (layer "F.Cu") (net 13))
 (segment (start 138.5 101.75) (end 140 103.25) (width 0.2) (layer "F.Cu") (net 13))
 (segment (start 138.725 99.025) (end 138.5 99.25) (width 0.2) (layer "F.Cu") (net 13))
 (segment (start 138.5 99.25) (end 138.5 101.75) (width 0.2) (layer "F.Cu") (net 13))
 (segment (start 151.11 102.54) (end 151.95 102.54) (width 0.2) (layer "F.Cu") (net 13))
 (segment (start 150.4 103.25) (end 151.11 102.54) (width 0.2) (layer "F.Cu") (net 13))
 (segment (start 135.4 100) (end 134.85 100) (width 0.2) (layer "F.Cu") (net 10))
 (segment (start 137.3625 99.675) (end 135.725 99.675) (width 0.2) (layer "F.Cu") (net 10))
 (segment (start 135.725 99.675) (end 135.4 100) (width 0.2) (layer "F.Cu") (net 10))
 (segment (start 136.325 100.325) (end 135.4 101.25) (width 0.2) (layer "F.Cu") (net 11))
 (segment (start 137.3625 100.325) (end 136.325 100.325) (width 0.2) (layer "F.Cu") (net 11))
 (segment (start 135.4 101.25) (end 134.85 101.25) (width 0.2) (layer "F.Cu") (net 11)))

